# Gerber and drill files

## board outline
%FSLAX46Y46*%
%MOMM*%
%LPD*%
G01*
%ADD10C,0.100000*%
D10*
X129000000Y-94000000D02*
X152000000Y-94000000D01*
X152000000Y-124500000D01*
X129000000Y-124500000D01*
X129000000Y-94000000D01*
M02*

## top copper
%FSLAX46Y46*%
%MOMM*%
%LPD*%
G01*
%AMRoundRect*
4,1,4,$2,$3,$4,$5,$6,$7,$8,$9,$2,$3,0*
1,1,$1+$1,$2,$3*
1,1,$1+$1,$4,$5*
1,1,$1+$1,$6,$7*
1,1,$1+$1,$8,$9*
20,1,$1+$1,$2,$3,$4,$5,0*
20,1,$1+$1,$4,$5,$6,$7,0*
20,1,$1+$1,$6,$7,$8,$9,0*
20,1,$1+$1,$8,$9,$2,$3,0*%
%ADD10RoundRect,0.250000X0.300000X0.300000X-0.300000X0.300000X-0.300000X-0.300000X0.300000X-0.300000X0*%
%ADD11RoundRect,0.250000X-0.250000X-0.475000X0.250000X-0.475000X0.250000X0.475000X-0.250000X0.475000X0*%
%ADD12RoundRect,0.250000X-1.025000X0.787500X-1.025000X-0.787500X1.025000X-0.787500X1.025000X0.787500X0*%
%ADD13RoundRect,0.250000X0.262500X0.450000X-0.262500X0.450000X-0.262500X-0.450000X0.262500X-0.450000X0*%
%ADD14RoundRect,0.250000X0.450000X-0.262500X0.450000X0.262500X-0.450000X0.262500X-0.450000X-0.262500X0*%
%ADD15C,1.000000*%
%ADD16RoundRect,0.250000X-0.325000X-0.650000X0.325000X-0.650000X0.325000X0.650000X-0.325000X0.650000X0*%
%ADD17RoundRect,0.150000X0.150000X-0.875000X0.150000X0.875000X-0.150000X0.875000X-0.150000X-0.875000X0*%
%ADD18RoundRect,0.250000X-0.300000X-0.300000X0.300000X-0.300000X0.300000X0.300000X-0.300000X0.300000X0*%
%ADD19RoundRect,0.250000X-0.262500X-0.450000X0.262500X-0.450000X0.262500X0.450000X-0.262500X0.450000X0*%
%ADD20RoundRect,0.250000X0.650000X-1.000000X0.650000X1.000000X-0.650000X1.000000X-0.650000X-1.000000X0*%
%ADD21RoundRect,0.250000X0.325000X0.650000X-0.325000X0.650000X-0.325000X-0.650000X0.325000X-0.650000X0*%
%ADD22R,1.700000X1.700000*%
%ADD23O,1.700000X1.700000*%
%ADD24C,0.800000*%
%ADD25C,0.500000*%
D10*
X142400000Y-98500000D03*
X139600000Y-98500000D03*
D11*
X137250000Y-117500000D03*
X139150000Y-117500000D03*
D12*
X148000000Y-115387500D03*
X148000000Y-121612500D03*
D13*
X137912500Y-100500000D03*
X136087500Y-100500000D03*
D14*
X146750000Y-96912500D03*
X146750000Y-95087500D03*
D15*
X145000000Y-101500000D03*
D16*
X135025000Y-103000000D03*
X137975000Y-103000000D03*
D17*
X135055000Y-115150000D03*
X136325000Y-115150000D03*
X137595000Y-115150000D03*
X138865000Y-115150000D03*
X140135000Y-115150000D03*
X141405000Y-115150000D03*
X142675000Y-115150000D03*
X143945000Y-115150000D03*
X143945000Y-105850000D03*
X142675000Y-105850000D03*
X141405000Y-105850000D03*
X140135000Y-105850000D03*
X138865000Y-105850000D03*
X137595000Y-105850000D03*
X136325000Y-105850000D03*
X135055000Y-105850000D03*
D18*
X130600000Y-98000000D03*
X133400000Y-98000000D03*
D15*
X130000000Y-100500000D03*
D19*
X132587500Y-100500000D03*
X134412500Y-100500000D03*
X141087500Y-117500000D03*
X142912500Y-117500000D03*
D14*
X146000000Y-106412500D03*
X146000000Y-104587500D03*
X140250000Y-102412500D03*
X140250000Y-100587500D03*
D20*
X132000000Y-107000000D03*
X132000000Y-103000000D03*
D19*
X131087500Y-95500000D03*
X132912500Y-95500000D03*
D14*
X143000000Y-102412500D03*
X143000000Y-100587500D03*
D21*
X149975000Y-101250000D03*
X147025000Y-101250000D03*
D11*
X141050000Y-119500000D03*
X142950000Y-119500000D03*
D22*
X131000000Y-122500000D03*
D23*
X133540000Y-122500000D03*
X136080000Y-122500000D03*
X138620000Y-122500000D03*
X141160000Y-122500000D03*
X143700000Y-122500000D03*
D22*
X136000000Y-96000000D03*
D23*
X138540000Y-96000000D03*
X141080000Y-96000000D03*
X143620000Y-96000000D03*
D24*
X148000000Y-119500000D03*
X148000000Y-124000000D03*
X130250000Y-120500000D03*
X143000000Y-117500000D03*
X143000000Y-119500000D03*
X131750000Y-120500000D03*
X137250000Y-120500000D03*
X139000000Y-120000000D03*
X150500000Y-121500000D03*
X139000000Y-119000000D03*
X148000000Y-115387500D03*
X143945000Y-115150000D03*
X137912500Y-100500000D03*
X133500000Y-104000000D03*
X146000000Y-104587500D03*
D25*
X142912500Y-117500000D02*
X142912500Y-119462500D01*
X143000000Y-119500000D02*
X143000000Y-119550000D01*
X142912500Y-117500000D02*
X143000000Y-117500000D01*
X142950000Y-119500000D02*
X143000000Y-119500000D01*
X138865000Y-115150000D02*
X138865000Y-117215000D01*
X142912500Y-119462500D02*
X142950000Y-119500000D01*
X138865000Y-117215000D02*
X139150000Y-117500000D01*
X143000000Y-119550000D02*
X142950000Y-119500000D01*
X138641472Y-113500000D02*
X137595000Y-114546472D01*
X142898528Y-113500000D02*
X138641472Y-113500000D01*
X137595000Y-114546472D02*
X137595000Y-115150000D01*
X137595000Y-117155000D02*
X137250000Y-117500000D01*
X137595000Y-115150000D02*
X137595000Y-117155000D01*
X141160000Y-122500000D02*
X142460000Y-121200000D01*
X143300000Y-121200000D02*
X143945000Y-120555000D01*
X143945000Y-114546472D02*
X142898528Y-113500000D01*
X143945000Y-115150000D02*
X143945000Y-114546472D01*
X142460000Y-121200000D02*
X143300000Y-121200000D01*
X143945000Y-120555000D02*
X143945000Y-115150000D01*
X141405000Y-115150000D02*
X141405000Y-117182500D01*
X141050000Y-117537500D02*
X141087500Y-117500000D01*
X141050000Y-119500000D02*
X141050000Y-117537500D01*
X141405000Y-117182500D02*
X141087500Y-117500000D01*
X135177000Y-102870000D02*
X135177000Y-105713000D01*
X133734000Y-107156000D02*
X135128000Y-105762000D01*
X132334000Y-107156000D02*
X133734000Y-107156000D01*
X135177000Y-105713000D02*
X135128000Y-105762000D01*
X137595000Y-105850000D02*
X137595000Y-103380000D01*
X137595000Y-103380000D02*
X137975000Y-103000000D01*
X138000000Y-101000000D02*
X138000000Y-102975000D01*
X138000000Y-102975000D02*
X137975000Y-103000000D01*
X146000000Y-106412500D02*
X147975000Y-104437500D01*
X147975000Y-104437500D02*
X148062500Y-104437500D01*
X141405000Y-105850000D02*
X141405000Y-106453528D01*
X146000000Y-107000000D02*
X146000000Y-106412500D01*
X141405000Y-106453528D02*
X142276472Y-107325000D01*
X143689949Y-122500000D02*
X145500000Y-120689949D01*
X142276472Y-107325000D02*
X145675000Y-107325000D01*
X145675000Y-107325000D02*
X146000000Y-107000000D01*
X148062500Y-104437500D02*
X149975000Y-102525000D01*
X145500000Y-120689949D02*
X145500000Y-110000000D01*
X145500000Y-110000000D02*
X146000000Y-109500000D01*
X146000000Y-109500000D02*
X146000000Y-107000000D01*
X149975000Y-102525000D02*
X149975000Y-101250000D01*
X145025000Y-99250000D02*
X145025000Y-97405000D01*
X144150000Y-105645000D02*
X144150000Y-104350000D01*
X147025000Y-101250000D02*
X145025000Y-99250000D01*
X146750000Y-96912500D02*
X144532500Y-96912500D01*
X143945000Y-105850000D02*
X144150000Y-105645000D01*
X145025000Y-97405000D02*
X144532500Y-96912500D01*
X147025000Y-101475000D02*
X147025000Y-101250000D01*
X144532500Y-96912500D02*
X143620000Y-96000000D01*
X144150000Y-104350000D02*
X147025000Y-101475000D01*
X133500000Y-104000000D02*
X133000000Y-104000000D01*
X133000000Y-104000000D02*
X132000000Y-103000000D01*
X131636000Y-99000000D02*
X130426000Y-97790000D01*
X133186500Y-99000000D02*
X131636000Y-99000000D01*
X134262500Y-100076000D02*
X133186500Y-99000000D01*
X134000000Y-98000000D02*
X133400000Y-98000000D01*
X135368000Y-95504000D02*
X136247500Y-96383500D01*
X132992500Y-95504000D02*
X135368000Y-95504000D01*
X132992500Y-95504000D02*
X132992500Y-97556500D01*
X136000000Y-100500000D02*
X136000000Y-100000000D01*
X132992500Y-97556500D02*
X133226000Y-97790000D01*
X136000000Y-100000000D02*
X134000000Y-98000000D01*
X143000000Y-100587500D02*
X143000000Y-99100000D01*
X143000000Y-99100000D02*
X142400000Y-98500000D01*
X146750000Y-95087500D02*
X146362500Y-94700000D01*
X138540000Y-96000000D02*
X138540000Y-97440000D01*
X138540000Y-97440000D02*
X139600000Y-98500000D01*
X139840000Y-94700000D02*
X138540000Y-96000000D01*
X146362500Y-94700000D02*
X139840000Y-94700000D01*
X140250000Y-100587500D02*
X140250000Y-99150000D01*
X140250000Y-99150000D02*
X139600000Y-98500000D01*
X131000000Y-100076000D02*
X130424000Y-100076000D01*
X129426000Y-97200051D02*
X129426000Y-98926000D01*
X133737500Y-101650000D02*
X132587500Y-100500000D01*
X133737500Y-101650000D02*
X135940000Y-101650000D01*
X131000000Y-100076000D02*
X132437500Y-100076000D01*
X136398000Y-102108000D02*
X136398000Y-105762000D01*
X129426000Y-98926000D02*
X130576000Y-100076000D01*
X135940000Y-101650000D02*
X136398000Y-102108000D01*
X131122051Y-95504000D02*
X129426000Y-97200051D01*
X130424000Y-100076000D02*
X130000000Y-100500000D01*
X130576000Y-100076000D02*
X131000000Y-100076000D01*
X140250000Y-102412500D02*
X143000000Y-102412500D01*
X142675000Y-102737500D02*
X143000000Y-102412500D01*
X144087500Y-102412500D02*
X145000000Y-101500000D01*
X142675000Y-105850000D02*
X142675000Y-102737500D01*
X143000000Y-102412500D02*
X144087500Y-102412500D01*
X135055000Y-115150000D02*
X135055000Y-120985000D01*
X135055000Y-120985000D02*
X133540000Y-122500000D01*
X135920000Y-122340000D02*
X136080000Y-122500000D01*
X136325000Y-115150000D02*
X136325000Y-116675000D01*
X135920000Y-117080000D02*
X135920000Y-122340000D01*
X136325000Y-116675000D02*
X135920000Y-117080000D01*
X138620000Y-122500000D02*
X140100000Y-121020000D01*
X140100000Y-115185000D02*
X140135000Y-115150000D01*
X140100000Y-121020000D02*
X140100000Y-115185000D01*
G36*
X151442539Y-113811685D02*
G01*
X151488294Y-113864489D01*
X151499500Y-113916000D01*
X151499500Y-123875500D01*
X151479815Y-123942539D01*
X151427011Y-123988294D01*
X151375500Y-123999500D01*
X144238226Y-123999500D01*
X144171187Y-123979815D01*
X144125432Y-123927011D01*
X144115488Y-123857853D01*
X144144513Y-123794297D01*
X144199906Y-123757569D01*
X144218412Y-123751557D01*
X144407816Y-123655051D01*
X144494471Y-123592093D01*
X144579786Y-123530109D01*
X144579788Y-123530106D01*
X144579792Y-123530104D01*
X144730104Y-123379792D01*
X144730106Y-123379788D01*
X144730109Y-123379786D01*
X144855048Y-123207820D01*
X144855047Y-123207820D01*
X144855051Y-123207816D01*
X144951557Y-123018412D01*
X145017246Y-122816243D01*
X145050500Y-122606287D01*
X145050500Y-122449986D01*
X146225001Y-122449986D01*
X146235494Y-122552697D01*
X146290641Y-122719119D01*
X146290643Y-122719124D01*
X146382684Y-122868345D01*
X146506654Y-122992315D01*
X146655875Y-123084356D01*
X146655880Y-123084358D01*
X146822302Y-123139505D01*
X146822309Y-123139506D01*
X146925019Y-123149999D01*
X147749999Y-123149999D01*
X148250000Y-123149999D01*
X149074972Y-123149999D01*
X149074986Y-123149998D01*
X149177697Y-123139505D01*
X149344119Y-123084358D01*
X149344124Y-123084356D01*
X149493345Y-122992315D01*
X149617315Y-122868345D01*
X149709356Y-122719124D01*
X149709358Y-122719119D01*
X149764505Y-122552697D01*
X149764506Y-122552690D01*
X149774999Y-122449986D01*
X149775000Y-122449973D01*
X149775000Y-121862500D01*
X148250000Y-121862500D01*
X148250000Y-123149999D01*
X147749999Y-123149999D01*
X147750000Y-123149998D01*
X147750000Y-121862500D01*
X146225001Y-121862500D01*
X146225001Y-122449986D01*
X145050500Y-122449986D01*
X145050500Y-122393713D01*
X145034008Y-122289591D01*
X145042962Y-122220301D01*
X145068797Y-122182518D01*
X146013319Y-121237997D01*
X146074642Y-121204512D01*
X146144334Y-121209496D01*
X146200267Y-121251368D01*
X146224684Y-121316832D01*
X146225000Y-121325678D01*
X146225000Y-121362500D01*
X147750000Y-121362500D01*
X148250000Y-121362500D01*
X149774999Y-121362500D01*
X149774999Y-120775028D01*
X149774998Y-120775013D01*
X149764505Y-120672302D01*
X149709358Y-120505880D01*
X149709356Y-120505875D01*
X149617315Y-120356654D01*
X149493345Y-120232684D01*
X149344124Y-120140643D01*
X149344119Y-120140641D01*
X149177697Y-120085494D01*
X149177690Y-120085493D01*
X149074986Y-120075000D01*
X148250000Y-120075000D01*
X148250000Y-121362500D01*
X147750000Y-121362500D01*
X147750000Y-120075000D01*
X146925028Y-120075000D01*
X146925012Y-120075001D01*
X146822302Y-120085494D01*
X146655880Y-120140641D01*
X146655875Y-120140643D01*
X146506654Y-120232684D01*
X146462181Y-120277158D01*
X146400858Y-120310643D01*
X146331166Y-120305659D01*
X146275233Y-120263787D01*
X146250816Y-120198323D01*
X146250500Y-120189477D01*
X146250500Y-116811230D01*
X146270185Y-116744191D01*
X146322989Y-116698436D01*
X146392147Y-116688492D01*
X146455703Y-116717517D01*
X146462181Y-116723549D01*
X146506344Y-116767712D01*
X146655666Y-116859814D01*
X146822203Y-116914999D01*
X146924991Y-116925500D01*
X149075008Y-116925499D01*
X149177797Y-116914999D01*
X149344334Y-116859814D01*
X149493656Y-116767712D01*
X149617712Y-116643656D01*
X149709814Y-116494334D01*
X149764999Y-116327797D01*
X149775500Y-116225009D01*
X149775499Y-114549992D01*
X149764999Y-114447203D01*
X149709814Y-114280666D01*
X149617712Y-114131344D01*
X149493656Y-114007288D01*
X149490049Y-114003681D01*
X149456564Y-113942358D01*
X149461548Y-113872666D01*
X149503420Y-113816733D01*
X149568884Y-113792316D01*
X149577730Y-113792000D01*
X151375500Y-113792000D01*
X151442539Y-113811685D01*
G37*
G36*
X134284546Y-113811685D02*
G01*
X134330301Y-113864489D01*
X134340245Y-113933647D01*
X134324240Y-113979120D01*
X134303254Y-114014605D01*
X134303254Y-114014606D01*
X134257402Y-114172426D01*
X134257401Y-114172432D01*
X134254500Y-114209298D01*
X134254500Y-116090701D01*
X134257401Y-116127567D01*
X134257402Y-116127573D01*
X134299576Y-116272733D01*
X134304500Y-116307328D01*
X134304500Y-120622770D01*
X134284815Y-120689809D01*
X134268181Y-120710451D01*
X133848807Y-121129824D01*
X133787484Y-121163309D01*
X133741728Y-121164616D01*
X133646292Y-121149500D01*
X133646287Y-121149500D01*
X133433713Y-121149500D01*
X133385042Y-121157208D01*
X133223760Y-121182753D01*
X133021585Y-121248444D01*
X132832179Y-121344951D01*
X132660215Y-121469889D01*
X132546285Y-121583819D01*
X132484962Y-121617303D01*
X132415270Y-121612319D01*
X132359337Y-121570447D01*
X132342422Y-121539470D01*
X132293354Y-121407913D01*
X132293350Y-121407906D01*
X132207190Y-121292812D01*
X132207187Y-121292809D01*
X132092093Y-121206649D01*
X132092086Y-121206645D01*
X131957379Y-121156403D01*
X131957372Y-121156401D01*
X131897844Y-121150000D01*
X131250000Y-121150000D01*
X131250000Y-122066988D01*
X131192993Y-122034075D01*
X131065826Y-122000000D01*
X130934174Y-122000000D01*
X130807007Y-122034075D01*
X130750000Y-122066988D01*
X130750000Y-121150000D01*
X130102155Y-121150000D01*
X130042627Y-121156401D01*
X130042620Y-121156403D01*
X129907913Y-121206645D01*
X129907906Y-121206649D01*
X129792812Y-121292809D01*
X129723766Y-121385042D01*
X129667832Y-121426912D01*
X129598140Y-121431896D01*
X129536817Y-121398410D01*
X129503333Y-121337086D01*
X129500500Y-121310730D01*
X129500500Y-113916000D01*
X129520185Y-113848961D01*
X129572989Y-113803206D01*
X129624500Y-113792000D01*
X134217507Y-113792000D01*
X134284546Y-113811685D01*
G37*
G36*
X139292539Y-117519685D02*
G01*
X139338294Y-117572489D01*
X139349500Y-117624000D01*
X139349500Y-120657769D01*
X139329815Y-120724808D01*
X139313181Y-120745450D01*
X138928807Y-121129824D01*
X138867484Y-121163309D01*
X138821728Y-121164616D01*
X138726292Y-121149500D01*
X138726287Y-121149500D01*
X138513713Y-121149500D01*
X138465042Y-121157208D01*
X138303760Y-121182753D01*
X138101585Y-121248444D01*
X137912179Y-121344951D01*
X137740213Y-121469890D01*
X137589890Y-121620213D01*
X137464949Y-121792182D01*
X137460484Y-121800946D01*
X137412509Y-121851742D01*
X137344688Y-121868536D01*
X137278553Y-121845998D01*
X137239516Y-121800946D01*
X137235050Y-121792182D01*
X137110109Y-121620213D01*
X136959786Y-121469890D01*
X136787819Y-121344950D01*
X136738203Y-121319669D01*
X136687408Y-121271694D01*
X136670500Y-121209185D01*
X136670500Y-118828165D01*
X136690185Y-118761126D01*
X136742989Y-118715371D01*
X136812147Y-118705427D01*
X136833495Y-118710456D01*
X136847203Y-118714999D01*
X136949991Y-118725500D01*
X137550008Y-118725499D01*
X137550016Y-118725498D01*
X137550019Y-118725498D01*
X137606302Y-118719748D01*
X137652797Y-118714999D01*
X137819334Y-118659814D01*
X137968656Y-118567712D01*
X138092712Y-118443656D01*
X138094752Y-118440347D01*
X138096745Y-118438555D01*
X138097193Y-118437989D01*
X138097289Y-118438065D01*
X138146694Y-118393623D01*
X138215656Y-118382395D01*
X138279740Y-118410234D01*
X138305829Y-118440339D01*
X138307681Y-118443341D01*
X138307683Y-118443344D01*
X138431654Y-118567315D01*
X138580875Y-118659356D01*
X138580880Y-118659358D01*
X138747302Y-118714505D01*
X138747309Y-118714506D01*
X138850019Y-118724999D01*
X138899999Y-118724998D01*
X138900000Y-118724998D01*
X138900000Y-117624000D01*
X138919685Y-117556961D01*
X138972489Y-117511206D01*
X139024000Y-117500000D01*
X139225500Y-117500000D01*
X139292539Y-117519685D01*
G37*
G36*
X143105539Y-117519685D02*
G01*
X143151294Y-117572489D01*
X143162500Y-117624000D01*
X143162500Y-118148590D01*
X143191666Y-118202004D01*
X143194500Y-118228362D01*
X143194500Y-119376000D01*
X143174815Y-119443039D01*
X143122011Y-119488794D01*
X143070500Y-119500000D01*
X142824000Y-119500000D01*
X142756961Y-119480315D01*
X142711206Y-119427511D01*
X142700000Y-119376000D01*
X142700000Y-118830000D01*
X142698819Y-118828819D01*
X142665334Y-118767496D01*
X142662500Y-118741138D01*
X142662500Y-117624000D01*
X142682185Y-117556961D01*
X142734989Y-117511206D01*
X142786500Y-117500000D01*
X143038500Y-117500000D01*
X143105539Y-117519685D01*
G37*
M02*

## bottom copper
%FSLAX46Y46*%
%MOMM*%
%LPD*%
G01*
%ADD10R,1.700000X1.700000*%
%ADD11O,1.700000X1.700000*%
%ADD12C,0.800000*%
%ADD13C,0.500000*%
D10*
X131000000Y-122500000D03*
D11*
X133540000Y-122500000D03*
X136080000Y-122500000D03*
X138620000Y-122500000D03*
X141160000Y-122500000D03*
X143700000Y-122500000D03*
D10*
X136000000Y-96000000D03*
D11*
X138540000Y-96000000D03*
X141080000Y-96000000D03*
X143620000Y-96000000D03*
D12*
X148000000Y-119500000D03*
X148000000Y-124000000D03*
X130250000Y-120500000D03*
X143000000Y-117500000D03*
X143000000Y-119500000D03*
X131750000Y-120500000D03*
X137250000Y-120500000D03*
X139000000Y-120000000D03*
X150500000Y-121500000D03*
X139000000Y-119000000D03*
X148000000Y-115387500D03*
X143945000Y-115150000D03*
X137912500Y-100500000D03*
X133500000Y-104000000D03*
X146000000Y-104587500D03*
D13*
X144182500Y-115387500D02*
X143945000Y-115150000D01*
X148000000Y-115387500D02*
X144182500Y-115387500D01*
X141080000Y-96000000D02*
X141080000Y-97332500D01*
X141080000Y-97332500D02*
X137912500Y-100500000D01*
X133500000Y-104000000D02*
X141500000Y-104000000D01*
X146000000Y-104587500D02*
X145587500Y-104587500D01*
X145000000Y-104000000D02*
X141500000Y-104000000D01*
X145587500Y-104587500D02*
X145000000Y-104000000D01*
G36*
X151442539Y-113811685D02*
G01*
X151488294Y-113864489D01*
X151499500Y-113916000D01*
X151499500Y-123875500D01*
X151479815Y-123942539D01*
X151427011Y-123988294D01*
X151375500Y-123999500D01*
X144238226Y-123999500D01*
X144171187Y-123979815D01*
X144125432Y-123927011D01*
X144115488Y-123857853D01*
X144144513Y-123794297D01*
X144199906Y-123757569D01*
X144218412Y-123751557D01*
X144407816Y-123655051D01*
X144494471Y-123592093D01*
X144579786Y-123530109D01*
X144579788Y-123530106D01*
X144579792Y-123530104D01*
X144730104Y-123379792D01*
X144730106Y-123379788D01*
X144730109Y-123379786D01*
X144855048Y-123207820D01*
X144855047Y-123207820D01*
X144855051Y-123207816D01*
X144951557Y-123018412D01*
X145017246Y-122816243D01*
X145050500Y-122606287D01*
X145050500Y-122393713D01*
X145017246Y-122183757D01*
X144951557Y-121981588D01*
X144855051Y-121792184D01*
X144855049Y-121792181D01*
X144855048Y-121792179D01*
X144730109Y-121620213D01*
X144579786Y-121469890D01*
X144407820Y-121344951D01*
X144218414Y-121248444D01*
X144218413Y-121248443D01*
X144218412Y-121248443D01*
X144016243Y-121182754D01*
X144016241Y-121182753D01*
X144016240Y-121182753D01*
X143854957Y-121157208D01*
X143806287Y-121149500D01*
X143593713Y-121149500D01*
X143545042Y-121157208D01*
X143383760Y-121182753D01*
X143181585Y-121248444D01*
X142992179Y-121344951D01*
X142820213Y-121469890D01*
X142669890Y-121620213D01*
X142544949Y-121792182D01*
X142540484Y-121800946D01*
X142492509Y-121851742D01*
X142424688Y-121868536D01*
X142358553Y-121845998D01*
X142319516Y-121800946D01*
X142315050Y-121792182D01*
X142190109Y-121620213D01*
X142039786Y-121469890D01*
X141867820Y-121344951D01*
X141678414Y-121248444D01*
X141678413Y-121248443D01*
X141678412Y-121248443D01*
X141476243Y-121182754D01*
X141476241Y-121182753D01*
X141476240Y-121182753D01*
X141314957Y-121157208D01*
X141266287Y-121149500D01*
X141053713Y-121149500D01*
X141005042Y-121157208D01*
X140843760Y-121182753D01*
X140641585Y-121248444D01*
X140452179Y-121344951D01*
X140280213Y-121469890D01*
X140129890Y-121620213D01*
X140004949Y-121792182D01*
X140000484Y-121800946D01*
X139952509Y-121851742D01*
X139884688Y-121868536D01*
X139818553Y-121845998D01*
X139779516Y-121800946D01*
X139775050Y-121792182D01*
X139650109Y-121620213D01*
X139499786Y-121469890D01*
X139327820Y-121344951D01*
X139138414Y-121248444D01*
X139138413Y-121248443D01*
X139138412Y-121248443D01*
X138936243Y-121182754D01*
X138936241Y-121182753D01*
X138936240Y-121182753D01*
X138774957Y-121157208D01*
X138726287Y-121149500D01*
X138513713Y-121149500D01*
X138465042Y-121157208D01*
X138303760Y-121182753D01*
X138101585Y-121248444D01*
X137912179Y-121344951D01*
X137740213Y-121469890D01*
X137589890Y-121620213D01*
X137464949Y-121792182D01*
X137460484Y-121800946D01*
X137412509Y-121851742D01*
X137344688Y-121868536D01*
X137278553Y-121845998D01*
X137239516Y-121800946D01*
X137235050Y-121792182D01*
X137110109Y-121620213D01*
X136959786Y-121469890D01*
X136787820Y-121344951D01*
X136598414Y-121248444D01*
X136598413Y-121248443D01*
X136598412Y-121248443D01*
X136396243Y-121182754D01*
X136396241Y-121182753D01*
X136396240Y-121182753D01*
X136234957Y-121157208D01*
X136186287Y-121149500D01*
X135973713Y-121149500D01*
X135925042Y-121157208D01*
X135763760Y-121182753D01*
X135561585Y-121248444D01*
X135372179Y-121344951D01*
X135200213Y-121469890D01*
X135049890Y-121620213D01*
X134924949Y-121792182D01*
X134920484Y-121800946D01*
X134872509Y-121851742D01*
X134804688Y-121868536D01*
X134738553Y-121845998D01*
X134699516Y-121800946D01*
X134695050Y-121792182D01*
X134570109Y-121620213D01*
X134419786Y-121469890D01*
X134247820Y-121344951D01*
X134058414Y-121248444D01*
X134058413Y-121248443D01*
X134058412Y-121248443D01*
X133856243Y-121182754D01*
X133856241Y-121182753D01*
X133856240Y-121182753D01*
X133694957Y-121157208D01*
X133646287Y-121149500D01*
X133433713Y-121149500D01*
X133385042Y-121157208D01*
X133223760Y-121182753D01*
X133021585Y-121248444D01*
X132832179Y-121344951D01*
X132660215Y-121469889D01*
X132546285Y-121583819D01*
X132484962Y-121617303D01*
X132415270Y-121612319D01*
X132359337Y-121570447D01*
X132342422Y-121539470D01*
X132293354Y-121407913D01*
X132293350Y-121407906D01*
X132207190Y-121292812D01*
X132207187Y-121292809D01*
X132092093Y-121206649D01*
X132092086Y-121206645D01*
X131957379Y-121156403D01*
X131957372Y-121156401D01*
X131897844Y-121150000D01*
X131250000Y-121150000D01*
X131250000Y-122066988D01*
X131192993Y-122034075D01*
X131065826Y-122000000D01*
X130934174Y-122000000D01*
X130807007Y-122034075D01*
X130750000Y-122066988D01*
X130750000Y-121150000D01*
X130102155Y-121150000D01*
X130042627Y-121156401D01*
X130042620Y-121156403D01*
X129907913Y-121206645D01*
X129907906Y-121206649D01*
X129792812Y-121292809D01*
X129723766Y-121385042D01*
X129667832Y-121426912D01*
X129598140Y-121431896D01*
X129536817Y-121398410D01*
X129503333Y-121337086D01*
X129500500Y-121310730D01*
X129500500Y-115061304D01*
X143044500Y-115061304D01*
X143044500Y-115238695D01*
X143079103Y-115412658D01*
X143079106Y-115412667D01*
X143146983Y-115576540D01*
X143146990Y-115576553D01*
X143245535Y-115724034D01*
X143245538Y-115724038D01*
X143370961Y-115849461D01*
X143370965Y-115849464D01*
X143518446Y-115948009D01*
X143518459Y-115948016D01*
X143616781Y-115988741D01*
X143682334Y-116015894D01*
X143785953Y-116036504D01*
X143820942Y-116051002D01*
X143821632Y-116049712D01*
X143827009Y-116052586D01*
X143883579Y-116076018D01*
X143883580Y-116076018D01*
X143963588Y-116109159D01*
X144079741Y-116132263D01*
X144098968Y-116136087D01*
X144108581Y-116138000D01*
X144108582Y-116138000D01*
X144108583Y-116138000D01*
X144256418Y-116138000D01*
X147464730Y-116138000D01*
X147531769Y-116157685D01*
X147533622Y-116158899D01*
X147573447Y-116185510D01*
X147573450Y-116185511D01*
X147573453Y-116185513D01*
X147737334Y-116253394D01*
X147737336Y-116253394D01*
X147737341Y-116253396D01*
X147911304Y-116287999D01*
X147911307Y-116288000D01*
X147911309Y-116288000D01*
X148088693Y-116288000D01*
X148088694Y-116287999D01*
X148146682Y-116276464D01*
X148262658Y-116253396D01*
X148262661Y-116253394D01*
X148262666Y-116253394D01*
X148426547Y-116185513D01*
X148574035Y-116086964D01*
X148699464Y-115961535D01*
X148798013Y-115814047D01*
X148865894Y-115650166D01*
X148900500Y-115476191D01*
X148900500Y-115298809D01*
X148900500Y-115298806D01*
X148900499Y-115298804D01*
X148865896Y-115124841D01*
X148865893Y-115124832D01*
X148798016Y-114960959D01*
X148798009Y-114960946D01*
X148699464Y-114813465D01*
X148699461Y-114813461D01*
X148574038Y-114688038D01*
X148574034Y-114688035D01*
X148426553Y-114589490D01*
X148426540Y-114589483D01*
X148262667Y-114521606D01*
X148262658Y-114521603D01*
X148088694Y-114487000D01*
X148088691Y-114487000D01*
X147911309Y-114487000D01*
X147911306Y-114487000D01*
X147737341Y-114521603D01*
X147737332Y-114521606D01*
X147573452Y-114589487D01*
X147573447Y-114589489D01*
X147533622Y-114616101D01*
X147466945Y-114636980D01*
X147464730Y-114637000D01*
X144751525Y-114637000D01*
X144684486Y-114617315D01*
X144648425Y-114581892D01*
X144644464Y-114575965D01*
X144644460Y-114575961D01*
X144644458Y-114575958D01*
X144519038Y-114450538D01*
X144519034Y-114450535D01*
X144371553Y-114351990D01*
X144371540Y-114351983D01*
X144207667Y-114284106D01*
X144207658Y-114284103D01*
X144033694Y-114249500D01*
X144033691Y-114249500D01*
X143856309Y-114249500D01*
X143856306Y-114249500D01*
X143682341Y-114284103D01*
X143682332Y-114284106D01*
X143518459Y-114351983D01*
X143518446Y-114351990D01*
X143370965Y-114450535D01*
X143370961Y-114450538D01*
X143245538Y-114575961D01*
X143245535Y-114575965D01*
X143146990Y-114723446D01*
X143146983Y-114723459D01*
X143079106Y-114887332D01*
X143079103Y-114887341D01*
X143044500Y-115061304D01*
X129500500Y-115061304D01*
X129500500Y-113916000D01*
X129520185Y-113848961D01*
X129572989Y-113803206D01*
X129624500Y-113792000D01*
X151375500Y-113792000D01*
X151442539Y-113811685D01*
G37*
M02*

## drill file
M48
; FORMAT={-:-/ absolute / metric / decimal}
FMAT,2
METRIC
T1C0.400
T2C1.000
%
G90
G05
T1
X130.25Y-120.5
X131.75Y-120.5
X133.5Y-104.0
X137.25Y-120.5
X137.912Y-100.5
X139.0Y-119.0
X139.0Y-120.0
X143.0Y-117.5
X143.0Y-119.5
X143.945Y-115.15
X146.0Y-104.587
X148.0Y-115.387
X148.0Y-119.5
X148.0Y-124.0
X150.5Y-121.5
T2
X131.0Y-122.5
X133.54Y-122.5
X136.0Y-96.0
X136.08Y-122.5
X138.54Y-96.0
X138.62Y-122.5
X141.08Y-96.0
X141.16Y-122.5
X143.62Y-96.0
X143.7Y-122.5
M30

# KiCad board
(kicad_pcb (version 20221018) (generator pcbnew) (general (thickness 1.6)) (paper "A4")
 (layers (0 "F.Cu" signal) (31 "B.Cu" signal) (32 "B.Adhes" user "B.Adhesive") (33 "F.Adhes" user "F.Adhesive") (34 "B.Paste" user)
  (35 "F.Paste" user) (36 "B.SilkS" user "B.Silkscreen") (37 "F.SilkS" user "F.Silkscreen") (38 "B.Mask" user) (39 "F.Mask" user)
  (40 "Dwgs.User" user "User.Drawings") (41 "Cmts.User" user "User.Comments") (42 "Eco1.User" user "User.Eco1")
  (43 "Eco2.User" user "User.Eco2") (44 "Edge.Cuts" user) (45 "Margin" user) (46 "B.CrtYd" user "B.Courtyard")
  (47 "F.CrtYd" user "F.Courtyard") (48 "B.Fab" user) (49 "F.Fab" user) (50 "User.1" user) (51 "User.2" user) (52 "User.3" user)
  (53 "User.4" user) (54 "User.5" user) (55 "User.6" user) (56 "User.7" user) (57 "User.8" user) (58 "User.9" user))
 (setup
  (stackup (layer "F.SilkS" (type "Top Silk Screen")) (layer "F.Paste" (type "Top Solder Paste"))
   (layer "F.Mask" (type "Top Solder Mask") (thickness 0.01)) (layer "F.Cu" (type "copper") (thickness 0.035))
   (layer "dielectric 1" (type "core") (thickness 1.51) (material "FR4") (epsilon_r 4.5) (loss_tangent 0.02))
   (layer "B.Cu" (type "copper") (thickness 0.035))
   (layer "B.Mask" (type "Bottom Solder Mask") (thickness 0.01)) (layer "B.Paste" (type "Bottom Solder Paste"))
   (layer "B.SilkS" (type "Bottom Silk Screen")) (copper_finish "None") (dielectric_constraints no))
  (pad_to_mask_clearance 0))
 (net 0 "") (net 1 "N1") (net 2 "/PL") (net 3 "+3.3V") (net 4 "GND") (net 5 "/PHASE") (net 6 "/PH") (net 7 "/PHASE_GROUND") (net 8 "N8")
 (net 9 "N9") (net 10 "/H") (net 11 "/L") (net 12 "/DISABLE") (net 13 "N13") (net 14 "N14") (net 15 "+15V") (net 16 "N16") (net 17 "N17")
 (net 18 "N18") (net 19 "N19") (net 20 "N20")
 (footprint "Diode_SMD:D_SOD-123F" (layer "F.Cu") (at 141 98.5 180)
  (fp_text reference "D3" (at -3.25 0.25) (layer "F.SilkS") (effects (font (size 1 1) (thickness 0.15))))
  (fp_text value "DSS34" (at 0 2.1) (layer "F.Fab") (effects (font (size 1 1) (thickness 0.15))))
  (pad "1" smd roundrect (at -1.4 0 180) (size 1.1 1.1) (layers "F.Cu" "F.Paste" "F.Mask") (roundrect_rratio 0.2272727273) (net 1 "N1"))
  (pad "2" smd roundrect (at 1.4 0 180) (size 1.1 1.1) (layers "F.Cu" "F.Paste" "F.Mask") (roundrect_rratio 0.2272727273) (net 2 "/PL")))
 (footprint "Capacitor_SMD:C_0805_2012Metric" (layer "F.Cu") (at 138.2 117.5)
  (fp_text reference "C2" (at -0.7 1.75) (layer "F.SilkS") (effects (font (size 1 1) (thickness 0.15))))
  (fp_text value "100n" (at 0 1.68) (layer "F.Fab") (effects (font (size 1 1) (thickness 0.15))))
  (pad "1" smd roundrect (at -0.95 0) (size 1 1.45) (layers "F.Cu" "F.Paste" "F.Mask") (roundrect_rratio 0.25) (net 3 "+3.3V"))
  (pad "2" smd roundrect (at 0.95 0) (size 1 1.45) (layers "F.Cu" "F.Paste" "F.Mask") (roundrect_rratio 0.25) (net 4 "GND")))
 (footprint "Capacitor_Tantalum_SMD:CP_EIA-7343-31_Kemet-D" (layer "F.Cu") (at 148 118.5 -90)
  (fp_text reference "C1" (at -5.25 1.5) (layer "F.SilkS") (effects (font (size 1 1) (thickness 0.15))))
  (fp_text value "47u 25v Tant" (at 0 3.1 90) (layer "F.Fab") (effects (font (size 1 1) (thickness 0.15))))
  (pad "1" smd roundrect (at -3.1125 0 270) (size 2.075 2.55) (layers "F.Cu" "F.Paste" "F.Mask") (roundrect_rratio 0.1204819277)
   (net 3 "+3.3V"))
  (pad "2" smd roundrect (at 3.1125 0 270) (size 2.075 2.55) (layers "F.Cu" "F.Paste" "F.Mask") (roundrect_rratio 0.1204819277)
   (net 4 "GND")))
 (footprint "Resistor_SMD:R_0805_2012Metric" (layer "F.Cu") (at 137 100.5 180)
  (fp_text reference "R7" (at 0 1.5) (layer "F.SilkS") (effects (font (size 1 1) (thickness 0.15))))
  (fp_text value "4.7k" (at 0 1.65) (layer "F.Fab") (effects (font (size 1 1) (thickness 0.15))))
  (pad "1" smd roundrect (at -0.9125 0 180) (size 1.025 1.4) (layers "F.Cu" "F.Paste" "F.Mask") (roundrect_rratio 0.243902439)
   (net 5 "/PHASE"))
  (pad "2" smd roundrect (at 0.9125 0 180) (size 1.025 1.4) (layers "F.Cu" "F.Paste" "F.Mask") (roundrect_rratio 0.243902439) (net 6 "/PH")))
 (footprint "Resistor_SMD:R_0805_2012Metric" (layer "F.Cu") (at 146.75 96 90)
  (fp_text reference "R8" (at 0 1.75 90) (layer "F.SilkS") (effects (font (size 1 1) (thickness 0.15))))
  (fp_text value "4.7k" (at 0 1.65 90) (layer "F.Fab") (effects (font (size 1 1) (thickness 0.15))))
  (pad "1" smd roundrect (at -0.9125 0 90) (size 1.025 1.4) (layers "F.Cu" "F.Paste" "F.Mask") (roundrect_rratio 0.243902439)
   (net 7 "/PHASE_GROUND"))
  (pad "2" smd roundrect (at 0.9125 0 90) (size 1.025 1.4) (layers "F.Cu" "F.Paste" "F.Mask") (roundrect_rratio 0.243902439) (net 2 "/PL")))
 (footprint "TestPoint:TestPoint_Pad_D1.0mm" (layer "F.Cu") (at 145 101.5)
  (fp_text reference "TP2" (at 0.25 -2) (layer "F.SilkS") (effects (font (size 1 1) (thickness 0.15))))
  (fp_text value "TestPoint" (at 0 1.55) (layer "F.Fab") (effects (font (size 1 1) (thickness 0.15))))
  (pad "1" smd circle (at 0 0) (size 1 1) (layers "F.Cu" "F.Mask") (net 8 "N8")))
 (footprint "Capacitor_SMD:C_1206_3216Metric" (layer "F.Cu") (at 136.5 103)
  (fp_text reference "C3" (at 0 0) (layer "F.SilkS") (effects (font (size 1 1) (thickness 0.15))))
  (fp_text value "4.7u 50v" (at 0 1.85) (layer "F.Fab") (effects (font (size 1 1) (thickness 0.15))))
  (pad "1" smd roundrect (at -1.475 0) (size 1.15 1.8) (layers "F.Cu" "F.Paste" "F.Mask") (roundrect_rratio 0.2173913043) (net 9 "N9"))
  (pad "2" smd roundrect (at 1.475 0) (size 1.15 1.8) (layers "F.Cu" "F.Paste" "F.Mask") (roundrect_rratio 0.2173913043) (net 5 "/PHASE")))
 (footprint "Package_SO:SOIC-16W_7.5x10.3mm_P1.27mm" (layer "F.Cu") (at 139.5 110.5 90)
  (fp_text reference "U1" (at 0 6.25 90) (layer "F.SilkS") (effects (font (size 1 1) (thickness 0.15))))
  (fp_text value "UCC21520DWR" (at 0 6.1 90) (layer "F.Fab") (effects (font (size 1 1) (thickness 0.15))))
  (pad "1" smd roundrect (at -4.65 -4.445 90) (size 2.05 0.6) (layers "F.Cu" "F.Paste" "F.Mask") (roundrect_rratio 0.25) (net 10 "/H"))
  (pad "2" smd roundrect (at -4.65 -3.175 90) (size 2.05 0.6) (layers "F.Cu" "F.Paste" "F.Mask") (roundrect_rratio 0.25) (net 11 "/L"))
  (pad "3" smd roundrect (at -4.65 -1.905 90) (size 2.05 0.6) (layers "F.Cu" "F.Paste" "F.Mask") (roundrect_rratio 0.25) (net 3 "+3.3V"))
  (pad "4" smd roundrect (at -4.65 -0.635 90) (size 2.05 0.6) (layers "F.Cu" "F.Paste" "F.Mask") (roundrect_rratio 0.25) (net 4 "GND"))
  (pad "5" smd roundrect (at -4.65 0.635 90) (size 2.05 0.6) (layers "F.Cu" "F.Paste" "F.Mask") (roundrect_rratio 0.25) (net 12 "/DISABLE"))
  (pad "6" smd roundrect (at -4.65 1.905 90) (size 2.05 0.6) (layers "F.Cu" "F.Paste" "F.Mask") (roundrect_rratio 0.25) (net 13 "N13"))
  (pad "7" smd roundrect (at -4.65 3.175 90) (size 2.05 0.6) (layers "F.Cu" "F.Paste" "F.Mask") (roundrect_rratio 0.25) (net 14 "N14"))
  (pad "8" smd roundrect (at -4.65 4.445 90) (size 2.05 0.6) (layers "F.Cu" "F.Paste" "F.Mask") (roundrect_rratio 0.25) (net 3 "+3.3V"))
  (pad "9" smd roundrect (at 4.65 4.445 90) (size 2.05 0.6) (layers "F.Cu" "F.Paste" "F.Mask") (roundrect_rratio 0.25)
   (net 7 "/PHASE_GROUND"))
  (pad "10" smd roundrect (at 4.65 3.175 90) (size 2.05 0.6) (layers "F.Cu" "F.Paste" "F.Mask") (roundrect_rratio 0.25) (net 8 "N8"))
  (pad "11" smd roundrect (at 4.65 1.905 90) (size 2.05 0.6) (layers "F.Cu" "F.Paste" "F.Mask") (roundrect_rratio 0.25) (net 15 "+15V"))
  (pad "12" smd roundrect (at 4.65 0.635 90) (size 2.05 0.6) (layers "F.Cu" "F.Paste" "F.Mask") (roundrect_rratio 0.25) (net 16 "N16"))
  (pad "13" smd roundrect (at 4.65 -0.635 90) (size 2.05 0.6) (layers "F.Cu" "F.Paste" "F.Mask") (roundrect_rratio 0.25) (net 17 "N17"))
  (pad "14" smd roundrect (at 4.65 -1.905 90) (size 2.05 0.6) (layers "F.Cu" "F.Paste" "F.Mask") (roundrect_rratio 0.25) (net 5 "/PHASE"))
  (pad "15" smd roundrect (at 4.65 -3.175 90) (size 2.05 0.6) (layers "F.Cu" "F.Paste" "F.Mask") (roundrect_rratio 0.25) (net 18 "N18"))
  (pad "16" smd roundrect (at 4.65 -4.445 90) (size 2.05 0.6) (layers "F.Cu" "F.Paste" "F.Mask") (roundrect_rratio 0.25) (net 9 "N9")))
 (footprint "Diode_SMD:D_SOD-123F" (layer "F.Cu") (at 132 98)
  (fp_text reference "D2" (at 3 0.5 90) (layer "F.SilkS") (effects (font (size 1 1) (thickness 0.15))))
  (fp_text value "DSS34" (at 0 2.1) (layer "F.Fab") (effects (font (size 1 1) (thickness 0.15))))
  (pad "1" smd roundrect (at -1.4 0) (size 1.1 1.1) (layers "F.Cu" "F.Paste" "F.Mask") (roundrect_rratio 0.2272727273) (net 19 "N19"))
  (pad "2" smd roundrect (at 1.4 0) (size 1.1 1.1) (layers "F.Cu" "F.Paste" "F.Mask") (roundrect_rratio 0.2272727273) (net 6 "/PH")))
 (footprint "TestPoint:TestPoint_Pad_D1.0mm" (layer "F.Cu") (at 130 100.5)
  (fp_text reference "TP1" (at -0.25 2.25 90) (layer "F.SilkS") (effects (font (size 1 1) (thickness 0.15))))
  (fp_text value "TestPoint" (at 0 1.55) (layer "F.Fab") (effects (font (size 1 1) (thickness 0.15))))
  (pad "1" smd circle (at 0 0) (size 1 1) (layers "F.Cu" "F.Mask") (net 18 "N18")))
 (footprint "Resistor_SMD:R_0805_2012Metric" (layer "F.Cu") (at 133.5 100.5)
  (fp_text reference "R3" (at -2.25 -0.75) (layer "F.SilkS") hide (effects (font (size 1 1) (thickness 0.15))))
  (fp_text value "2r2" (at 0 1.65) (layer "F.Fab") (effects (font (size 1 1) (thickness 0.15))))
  (pad "1" smd roundrect (at -0.9125 0) (size 1.025 1.4) (layers "F.Cu" "F.Paste" "F.Mask") (roundrect_rratio 0.243902439) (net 18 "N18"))
  (pad "2" smd roundrect (at 0.9125 0) (size 1.025 1.4) (layers "F.Cu" "F.Paste" "F.Mask") (roundrect_rratio 0.243902439) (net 19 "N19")))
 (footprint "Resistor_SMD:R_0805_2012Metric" (layer "F.Cu") (at 142 117.5)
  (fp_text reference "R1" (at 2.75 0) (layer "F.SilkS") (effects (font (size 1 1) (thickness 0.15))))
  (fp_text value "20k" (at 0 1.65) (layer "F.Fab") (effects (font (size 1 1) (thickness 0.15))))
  (pad "1" smd roundrect (at -0.9125 0) (size 1.025 1.4) (layers "F.Cu" "F.Paste" "F.Mask") (roundrect_rratio 0.243902439) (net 13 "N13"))
  (pad "2" smd roundrect (at 0.9125 0) (size 1.025 1.4) (layers "F.Cu" "F.Paste" "F.Mask") (roundrect_rratio 0.243902439) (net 4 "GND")))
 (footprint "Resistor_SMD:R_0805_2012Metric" (layer "F.Cu") (at 146 105.5 90)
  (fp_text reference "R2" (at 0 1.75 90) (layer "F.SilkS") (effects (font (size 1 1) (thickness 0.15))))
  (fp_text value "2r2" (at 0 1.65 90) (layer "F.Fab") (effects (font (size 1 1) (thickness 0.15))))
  (pad "1" smd roundrect (at -0.9125 0 90) (size 1.025 1.4) (layers "F.Cu" "F.Paste" "F.Mask") (roundrect_rratio 0.243902439)
   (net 15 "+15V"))
  (pad "2" smd roundrect (at 0.9125 0 90) (size 1.025 1.4) (layers "F.Cu" "F.Paste" "F.Mask") (roundrect_rratio 0.243902439) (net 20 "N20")))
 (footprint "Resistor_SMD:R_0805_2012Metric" (layer "F.Cu") (at 140.25 101.5 90)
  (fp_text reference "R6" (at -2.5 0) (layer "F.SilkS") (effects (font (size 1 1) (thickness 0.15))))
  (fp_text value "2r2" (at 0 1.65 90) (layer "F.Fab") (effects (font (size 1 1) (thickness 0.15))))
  (pad "1" smd roundrect (at -0.9125 0 90) (size 1.025 1.4) (layers "F.Cu" "F.Paste" "F.Mask") (roundrect_rratio 0.243902439) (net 8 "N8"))
  (pad "2" smd roundrect (at 0.9125 0 90) (size 1.025 1.4) (layers "F.Cu" "F.Paste" "F.Mask") (roundrect_rratio 0.243902439) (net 2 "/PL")))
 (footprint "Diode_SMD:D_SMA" (layer "F.Cu") (at 132 105 90)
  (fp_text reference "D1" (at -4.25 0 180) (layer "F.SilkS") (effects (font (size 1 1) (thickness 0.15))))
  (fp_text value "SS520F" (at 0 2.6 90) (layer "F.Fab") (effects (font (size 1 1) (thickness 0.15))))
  (pad "1" smd roundrect (at -2 0 90) (size 2.5 1.8) (layers "F.Cu" "F.Paste" "F.Mask") (roundrect_rratio 0.1388888889) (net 9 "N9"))
  (pad "2" smd roundrect (at 2 0 90) (size 2.5 1.8) (layers "F.Cu" "F.Paste" "F.Mask") (roundrect_rratio 0.1388888889) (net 20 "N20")))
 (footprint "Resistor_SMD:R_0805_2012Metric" (layer "F.Cu") (at 132 95.5)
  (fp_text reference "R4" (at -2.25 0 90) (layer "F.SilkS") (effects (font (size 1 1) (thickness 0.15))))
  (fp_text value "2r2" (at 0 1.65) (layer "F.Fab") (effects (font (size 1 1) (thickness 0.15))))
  (pad "1" smd roundrect (at -0.9125 0) (size 1.025 1.4) (layers "F.Cu" "F.Paste" "F.Mask") (roundrect_rratio 0.243902439) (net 18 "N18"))
  (pad "2" smd roundrect (at 0.9125 0) (size 1.025 1.4) (layers "F.Cu" "F.Paste" "F.Mask") (roundrect_rratio 0.243902439) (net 6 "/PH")))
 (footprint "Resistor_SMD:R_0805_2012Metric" (layer "F.Cu") (at 143 101.5 90)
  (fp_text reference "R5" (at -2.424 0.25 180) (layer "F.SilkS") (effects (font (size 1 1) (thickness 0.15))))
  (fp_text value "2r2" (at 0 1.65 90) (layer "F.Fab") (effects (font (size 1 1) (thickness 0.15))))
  (pad "1" smd roundrect (at -0.9125 0 90) (size 1.025 1.4) (layers "F.Cu" "F.Paste" "F.Mask") (roundrect_rratio 0.243902439) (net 8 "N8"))
  (pad "2" smd roundrect (at 0.9125 0 90) (size 1.025 1.4) (layers "F.Cu" "F.Paste" "F.Mask") (roundrect_rratio 0.243902439) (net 1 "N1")))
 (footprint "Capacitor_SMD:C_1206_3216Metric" (layer "F.Cu") (at 148.5 101.25 180)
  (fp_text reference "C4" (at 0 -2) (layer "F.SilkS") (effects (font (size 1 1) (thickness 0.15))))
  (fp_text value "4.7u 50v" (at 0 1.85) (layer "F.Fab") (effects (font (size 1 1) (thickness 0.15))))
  (pad "1" smd roundrect (at -1.475 0 180) (size 1.15 1.8) (layers "F.Cu" "F.Paste" "F.Mask") (roundrect_rratio 0.2173913043)
   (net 15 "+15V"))
  (pad "2" smd roundrect (at 1.475 0 180) (size 1.15 1.8) (layers "F.Cu" "F.Paste" "F.Mask") (roundrect_rratio 0.2173913043)
   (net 7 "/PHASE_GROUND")))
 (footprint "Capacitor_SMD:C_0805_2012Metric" (layer "F.Cu") (at 142 119.5)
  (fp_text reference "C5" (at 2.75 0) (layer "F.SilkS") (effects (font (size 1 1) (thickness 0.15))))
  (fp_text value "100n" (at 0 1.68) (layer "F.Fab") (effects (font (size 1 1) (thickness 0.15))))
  (pad "1" smd roundrect (at -0.95 0) (size 1 1.45) (layers "F.Cu" "F.Paste" "F.Mask") (roundrect_rratio 0.25) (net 13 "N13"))
  (pad "2" smd roundrect (at 0.95 0) (size 1 1.45) (layers "F.Cu" "F.Paste" "F.Mask") (roundrect_rratio 0.25) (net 4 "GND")))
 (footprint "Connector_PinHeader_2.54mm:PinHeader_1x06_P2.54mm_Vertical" (layer "B.Cu") (at 131 122.5 -90)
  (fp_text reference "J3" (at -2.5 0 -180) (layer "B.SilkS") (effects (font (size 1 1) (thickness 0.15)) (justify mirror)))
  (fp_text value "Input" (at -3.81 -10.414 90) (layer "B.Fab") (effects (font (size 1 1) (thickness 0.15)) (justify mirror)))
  (pad "1" thru_hole rect (at 0 0 270) (size 1.7 1.7) (drill 1) (layers "*.Cu" "*.Mask") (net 4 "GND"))
  (pad "2" thru_hole oval (at 0 -2.54 270) (size 1.7 1.7) (drill 1) (layers "*.Cu" "*.Mask") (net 10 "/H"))
  (pad "3" thru_hole oval (at 0 -5.08 270) (size 1.7 1.7) (drill 1) (layers "*.Cu" "*.Mask") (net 11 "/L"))
  (pad "4" thru_hole oval (at 0 -7.62 270) (size 1.7 1.7) (drill 1) (layers "*.Cu" "*.Mask") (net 12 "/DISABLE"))
  (pad "5" thru_hole oval (at 0 -10.16 270) (size 1.7 1.7) (drill 1) (layers "*.Cu" "*.Mask") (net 3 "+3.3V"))
  (pad "6" thru_hole oval (at 0 -12.7 270) (size 1.7 1.7) (drill 1) (layers "*.Cu" "*.Mask") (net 15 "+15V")))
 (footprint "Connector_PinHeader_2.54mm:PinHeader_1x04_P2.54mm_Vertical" (layer "B.Cu") (at 136 96 -90)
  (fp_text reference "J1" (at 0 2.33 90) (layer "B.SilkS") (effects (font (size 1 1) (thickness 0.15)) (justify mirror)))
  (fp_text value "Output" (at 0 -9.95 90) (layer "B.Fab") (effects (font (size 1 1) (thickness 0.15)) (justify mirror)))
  (pad "1" thru_hole rect (at 0 0 270) (size 1.7 1.7) (drill 1) (layers "*.Cu" "*.Mask") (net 6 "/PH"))
  (pad "2" thru_hole oval (at 0 -2.54 270) (size 1.7 1.7) (drill 1) (layers "*.Cu" "*.Mask") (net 2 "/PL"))
  (pad "3" thru_hole oval (at 0 -5.08 270) (size 1.7 1.7) (drill 1) (layers "*.Cu" "*.Mask") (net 5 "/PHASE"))
  (pad "4" thru_hole oval (at 0 -7.62 270) (size 1.7 1.7) (drill 1) (layers "*.Cu" "*.Mask") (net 7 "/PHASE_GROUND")))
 (gr_rect (start 129 94) (end 152 124.5) (stroke (width 0.1) (type default)) (fill none) (layer "Edge.Cuts"))
 (segment (start 142.9125 117.5) (end 142.9125 119.4625) (width 0.5) (layer "F.Cu") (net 4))
 (segment (start 143 119.5) (end 143 119.55) (width 0.5) (layer "F.Cu") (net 4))
 (segment (start 142.9125 117.5) (end 143 117.5) (width 0.5) (layer "F.Cu") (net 4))
 (segment (start 142.95 119.5) (end 143 119.5) (width 0.5) (layer "F.Cu") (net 4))
 (segment (start 138.865 115.15) (end 138.865 117.215) (width 0.5) (layer "F.Cu") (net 4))
 (segment (start 142.9125 119.4625) (end 142.95 119.5) (width 0.5) (layer "F.Cu") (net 4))
 (segment (start 138.865 117.215) (end 139.15 117.5) (width 0.5) (layer "F.Cu") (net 4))
 (segment (start 143 119.55) (end 142.95 119.5) (width 0.5) (layer "F.Cu") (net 4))
 (via (at 148 119.5) (size 0.8) (drill 0.4) (layers "F.Cu" "B.Cu") (free) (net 4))
 (via (at 148 124) (size 0.8) (drill 0.4) (layers "F.Cu" "B.Cu") (free) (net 4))
 (via (at 130.25 120.5) (size 0.8) (drill 0.4) (layers "F.Cu" "B.Cu") (free) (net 4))
 (via (at 143 117.5) (size 0.8) (drill 0.4) (layers "F.Cu" "B.Cu") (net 4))
 (via (at 143 119.5) (size 0.8) (drill 0.4) (layers "F.Cu" "B.Cu") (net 4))
 (via (at 131.75 120.5) (size 0.8) (drill 0.4) (layers "F.Cu" "B.Cu") (free) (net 4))
 (via (at 137.25 120.5) (size 0.8) (drill 0.4) (layers "F.Cu" "B.Cu") (free) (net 4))
 (via (at 139 120) (size 0.8) (drill 0.4) (layers "F.Cu" "B.Cu") (free) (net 4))
 (via (at 150.5 121.5) (size 0.8) (drill 0.4) (layers "F.Cu" "B.Cu") (free) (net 4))
 (via (at 139 119) (size 0.8) (drill 0.4) (layers "F.Cu" "B.Cu") (free) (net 4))
 (segment (start 138.641472 113.5) (end 137.595 114.546472) (width 0.5) (layer "F.Cu") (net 3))
 (segment (start 142.898528 113.5) (end 138.641472 113.5) (width 0.5) (layer "F.Cu") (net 3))
 (segment (start 137.595 114.546472) (end 137.595 115.15) (width 0.5) (layer "F.Cu") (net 3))
 (segment (start 137.595 117.155) (end 137.25 117.5) (width 0.5) (layer "F.Cu") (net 3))
 (segment (start 137.595 115.15) (end 137.595 117.155) (width 0.5) (layer "F.Cu") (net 3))
 (segment (start 141.16 122.5) (end 142.46 121.2) (width 0.5) (layer "F.Cu") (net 3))
 (segment (start 143.3 121.2) (end 143.945 120.555) (width 0.5) (layer "F.Cu") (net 3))
 (segment (start 143.945 114.546472) (end 142.898528 113.5) (width 0.5) (layer "F.Cu") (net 3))
 (segment (start 143.945 115.15) (end 143.945 114.546472) (width 0.5) (layer "F.Cu") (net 3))
 (segment (start 142.46 121.2) (end 143.3 121.2) (width 0.5) (layer "F.Cu") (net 3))
 (segment (start 143.945 120.555) (end 143.945 115.15) (width 0.5) (layer "F.Cu") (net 3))
 (via (at 148 115.3875) (size 0.8) (drill 0.4) (layers "F.Cu" "B.Cu") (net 3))
 (via (at 143.945 115.15) (size 0.8) (drill 0.4) (layers "F.Cu" "B.Cu") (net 3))
 (segment (start 144.1825 115.3875) (end 143.945 115.15) (width 0.5) (layer "B.Cu") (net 3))
 (segment (start 148 115.3875) (end 144.1825 115.3875) (width 0.5) (layer "B.Cu") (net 3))
 (segment (start 141.405 115.15) (end 141.405 117.1825) (width 0.5) (layer "F.Cu") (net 13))
 (segment (start 141.05 117.5375) (end 141.0875 117.5) (width 0.5) (layer "F.Cu") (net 13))
 (segment (start 141.05 119.5) (end 141.05 117.5375) (width 0.5) (layer "F.Cu") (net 13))
 (segment (start 141.405 117.1825) (end 141.0875 117.5) (width 0.5) (layer "F.Cu") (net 13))
 (segment (start 135.177 102.87) (end 135.177 105.713) (width 0.5) (layer "F.Cu") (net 9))
 (segment (start 133.734 107.156) (end 135.128 105.762) (width 0.5) (layer "F.Cu") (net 9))
 (segment (start 132.334 107.156) (end 133.734 107.156) (width 0.5) (layer "F.Cu") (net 9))
 (segment (start 135.177 105.713) (end 135.128 105.762) (width 0.5) (layer "F.Cu") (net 9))
 (segment (start 137.595 105.85) (end 137.595 103.38) (width 0.5) (layer "F.Cu") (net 5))
 (segment (start 137.595 103.38) (end 137.975 103) (width 0.5) (layer "F.Cu") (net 5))
 (segment (start 138 101) (end 138 102.975) (width 0.5) (layer "F.Cu") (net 5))
 (segment (start 138 102.975) (end 137.975 103) (width 0.5) (layer "F.Cu") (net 5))
 (via (at 137.9125 100.5) (size 0.8) (drill 0.4) (layers "F.Cu" "B.Cu") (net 5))
 (segment (start 141.08 96) (end 141.08 97.3325) (width 0.5) (layer "B.Cu") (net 5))
 (segment (start 141.08 97.3325) (end 137.9125 100.5) (width 0.5) (layer "B.Cu") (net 5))
 (segment (start 146 106.4125) (end 147.975 104.4375) (width 0.5) (layer "F.Cu") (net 15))
 (segment (start 147.975 104.4375) (end 148.0625 104.4375) (width 0.5) (layer "F.Cu") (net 15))
 (segment (start 141.405 105.85) (end 141.405 106.453528) (width 0.5) (layer "F.Cu") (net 15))
 (segment (start 146 107) (end 146 106.4125) (width 0.5) (layer "F.Cu") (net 15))
 (segment (start 141.405 106.453528) (end 142.276472 107.325) (width 0.5) (layer "F.Cu") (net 15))
 (segment (start 143.689949 122.5) (end 145.5 120.689949) (width 0.5) (layer "F.Cu") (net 15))
 (segment (start 142.276472 107.325) (end 145.675 107.325) (width 0.5) (layer "F.Cu") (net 15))
 (segment (start 145.675 107.325) (end 146 107) (width 0.5) (layer "F.Cu") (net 15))
 (segment (start 148.0625 104.4375) (end 149.975 102.525) (width 0.5) (layer "F.Cu") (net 15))
 (segment (start 145.5 120.689949) (end 145.5 110) (width 0.5) (layer "F.Cu") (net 15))
 (segment (start 145.5 110) (end 146 109.5) (width 0.5) (layer "F.Cu") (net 15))
 (segment (start 146 109.5) (end 146 107) (width 0.5) (layer "F.Cu") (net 15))
 (segment (start 149.975 102.525) (end 149.975 101.25) (width 0.5) (layer "F.Cu") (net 15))
 (segment (start 145.025 99.25) (end 145.025 97.405) (width 0.5) (layer "F.Cu") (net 7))
 (segment (start 144.15 105.645) (end 144.15 104.35) (width 0.5) (layer "F.Cu") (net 7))
 (segment (start 147.025 101.25) (end 145.025 99.25) (width 0.5) (layer "F.Cu") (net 7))
 (segment (start 146.75 96.9125) (end 144.5325 96.9125) (width 0.5) (layer "F.Cu") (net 7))
 (segment (start 143.945 105.85) (end 144.15 105.645) (width 0.5) (layer "F.Cu") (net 7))
 (segment (start 145.025 97.405) (end 144.5325 96.9125) (width 0.5) (layer "F.Cu") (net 7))
 (segment (start 147.025 101.475) (end 147.025 101.25) (width 0.5) (layer "F.Cu") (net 7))
 (segment (start 144.5325 96.9125) (end 143.62 96) (width 0.5) (layer "F.Cu") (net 7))
 (segment (start 144.15 104.35) (end 147.025 101.475) (width 0.5) (layer "F.Cu") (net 7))
 (segment (start 133.5 104) (end 133 104) (width 0.5) (layer "F.Cu") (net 20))
 (segment (start 133 104) (end 132 103) (width 0.5) (layer "F.Cu") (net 20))
 (via (at 133.5 104) (size 0.8) (drill 0.4) (layers "F.Cu" "B.Cu") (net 20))
 (via (at 146 104.5875) (size 0.8) (drill 0.4) (layers "F.Cu" "B.Cu") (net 20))
 (segment (start 133.5 104) (end 141.5 104) (width 0.5) (layer "B.Cu") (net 20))
 (segment (start 146 104.5875) (end 145.5875 104.5875) (width 0.5) (layer "B.Cu") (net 20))
 (segment (start 145 104) (end 141.5 104) (width 0.5) (layer "B.Cu") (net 20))
 (segment (start 145.5875 104.5875) (end 145 104) (width 0.5) (layer "B.Cu") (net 20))
 (segment (start 131.636 99) (end 130.426 97.79) (width 0.5) (layer "F.Cu") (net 19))
 (segment (start 133.1865 99) (end 131.636 99) (width 0.5) (layer "F.Cu") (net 19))
 (segment (start 134.2625 100.076) (end 133.1865 99) (width 0.5) (layer "F.Cu") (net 19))
 (segment (start 134 98) (end 133.4 98) (width 0.5) (layer "F.Cu") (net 6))
 (segment (start 135.368 95.504) (end 136.2475 96.3835) (width 0.5) (layer "F.Cu") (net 6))
 (segment (start 132.9925 95.504) (end 135.368 95.504) (width 0.5) (layer "F.Cu") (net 6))
 (segment (start 132.9925 95.504) (end 132.9925 97.5565) (width 0.5) (layer "F.Cu") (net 6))
 (segment (start 136 100.5) (end 136 100) (width 0.5) (layer "F.Cu") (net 6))
 (segment (start 132.9925 97.5565) (end 133.226 97.79) (width 0.5) (layer "F.Cu") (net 6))
 (segment (start 136 100) (end 134 98) (width 0.5) (layer "F.Cu") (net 6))
 (segment (start 143 100.5875) (end 143 99.1) (width 0.5) (layer "F.Cu") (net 1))
 (segment (start 143 99.1) (end 142.4 98.5) (width 0.5) (layer "F.Cu") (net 1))
 (segment (start 146.75 95.0875) (end 146.3625 94.7) (width 0.5) (layer "F.Cu") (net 2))
 (segment (start 138.54 96) (end 138.54 97.44) (width 0.5) (layer "F.Cu") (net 2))
 (segment (start 138.54 97.44) (end 139.6 98.5) (width 0.5) (layer "F.Cu") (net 2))
 (segment (start 139.84 94.7) (end 138.54 96) (width 0.5) (layer "F.Cu") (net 2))
 (segment (start 146.3625 94.7) (end 139.84 94.7) (width 0.5) (layer "F.Cu") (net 2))
 (segment (start 140.25 100.5875) (end 140.25 99.15) (width 0.5) (layer "F.Cu") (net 2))
 (segment (start 140.25 99.15) (end 139.6 98.5) (width 0.5) (layer "F.Cu") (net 2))
 (segment (start 131 100.076) (end 130.424 100.076) (width 0.5) (layer "F.Cu") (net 18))
 (segment (start 129.426 97.200051) (end 129.426 98.926) (width 0.5) (layer "F.Cu") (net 18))
 (segment (start 133.7375 101.65) (end 132.5875 100.5) (width 0.5) (layer "F.Cu") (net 18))
 (segment (start 133.7375 101.65) (end 135.94 101.65) (width 0.5) (layer "F.Cu") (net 18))
 (segment (start 131 100.076) (end 132.4375 100.076) (width 0.5) (layer "F.Cu") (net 18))
 (segment (start 136.398 102.108) (end 136.398 105.762) (width 0.5) (layer "F.Cu") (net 18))
 (segment (start 129.426 98.926) (end 130.576 100.076) (width 0.5) (layer "F.Cu") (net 18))
 (segment (start 135.94 101.65) (end 136.398 102.108) (width 0.5) (layer "F.Cu") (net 18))
 (segment (start 131.122051 95.504) (end 129.426 97.200051) (width 0.5) (layer "F.Cu") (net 18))
 (segment (start 130.424 100.076) (end 130 100.5) (width 0.5) (layer "F.Cu") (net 18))
 (segment (start 130.576 100.076) (end 131 100.076) (width 0.5) (layer "F.Cu") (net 18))
 (segment (start 140.25 102.4125) (end 143 102.4125) (width 0.5) (layer "F.Cu") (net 8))
 (segment (start 142.675 102.7375) (end 143 102.4125) (width 0.5) (layer "F.Cu") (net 8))
 (segment (start 144.0875 102.4125) (end 145 101.5) (width 0.5) (layer "F.Cu") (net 8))
 (segment (start 142.675 105.85) (end 142.675 102.7375) (width 0.5) (layer "F.Cu") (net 8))
 (segment (start 143 102.4125) (end 144.0875 102.4125) (width 0.5) (layer "F.Cu") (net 8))
 (segment (start 135.055 115.15) (end 135.055 120.985) (width 0.5) (layer "F.Cu") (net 10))
 (segment (start 135.055 120.985) (end 133.54 122.5) (width 0.5) (layer "F.Cu") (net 10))
 (segment (start 135.92 122.34) (end 136.08 122.5) (width 0.5) (layer "F.Cu") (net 11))
 (segment (start 136.325 115.15) (end 136.325 116.675) (width 0.5) (layer "F.Cu") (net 11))
 (segment (start 135.92 117.08) (end 135.92 122.34) (width 0.5) (layer "F.Cu") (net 11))
 (segment (start 136.325 116.675) (end 135.92 117.08) (width 0.5) (layer "F.Cu") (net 11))
 (segment (start 138.62 122.5) (end 140.1 121.02) (width 0.5) (layer "F.Cu") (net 12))
 (segment (start 140.1 115.185) (end 140.135 115.15) (width 0.5) (layer "F.Cu") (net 12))
 (segment (start 140.1 121.02) (end 140.1 115.185) (width 0.5) (layer "F.Cu") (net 12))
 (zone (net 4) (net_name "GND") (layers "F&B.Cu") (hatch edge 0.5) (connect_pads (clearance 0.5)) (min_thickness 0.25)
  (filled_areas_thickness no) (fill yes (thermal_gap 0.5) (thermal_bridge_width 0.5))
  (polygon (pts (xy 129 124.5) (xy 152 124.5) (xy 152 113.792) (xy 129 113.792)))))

